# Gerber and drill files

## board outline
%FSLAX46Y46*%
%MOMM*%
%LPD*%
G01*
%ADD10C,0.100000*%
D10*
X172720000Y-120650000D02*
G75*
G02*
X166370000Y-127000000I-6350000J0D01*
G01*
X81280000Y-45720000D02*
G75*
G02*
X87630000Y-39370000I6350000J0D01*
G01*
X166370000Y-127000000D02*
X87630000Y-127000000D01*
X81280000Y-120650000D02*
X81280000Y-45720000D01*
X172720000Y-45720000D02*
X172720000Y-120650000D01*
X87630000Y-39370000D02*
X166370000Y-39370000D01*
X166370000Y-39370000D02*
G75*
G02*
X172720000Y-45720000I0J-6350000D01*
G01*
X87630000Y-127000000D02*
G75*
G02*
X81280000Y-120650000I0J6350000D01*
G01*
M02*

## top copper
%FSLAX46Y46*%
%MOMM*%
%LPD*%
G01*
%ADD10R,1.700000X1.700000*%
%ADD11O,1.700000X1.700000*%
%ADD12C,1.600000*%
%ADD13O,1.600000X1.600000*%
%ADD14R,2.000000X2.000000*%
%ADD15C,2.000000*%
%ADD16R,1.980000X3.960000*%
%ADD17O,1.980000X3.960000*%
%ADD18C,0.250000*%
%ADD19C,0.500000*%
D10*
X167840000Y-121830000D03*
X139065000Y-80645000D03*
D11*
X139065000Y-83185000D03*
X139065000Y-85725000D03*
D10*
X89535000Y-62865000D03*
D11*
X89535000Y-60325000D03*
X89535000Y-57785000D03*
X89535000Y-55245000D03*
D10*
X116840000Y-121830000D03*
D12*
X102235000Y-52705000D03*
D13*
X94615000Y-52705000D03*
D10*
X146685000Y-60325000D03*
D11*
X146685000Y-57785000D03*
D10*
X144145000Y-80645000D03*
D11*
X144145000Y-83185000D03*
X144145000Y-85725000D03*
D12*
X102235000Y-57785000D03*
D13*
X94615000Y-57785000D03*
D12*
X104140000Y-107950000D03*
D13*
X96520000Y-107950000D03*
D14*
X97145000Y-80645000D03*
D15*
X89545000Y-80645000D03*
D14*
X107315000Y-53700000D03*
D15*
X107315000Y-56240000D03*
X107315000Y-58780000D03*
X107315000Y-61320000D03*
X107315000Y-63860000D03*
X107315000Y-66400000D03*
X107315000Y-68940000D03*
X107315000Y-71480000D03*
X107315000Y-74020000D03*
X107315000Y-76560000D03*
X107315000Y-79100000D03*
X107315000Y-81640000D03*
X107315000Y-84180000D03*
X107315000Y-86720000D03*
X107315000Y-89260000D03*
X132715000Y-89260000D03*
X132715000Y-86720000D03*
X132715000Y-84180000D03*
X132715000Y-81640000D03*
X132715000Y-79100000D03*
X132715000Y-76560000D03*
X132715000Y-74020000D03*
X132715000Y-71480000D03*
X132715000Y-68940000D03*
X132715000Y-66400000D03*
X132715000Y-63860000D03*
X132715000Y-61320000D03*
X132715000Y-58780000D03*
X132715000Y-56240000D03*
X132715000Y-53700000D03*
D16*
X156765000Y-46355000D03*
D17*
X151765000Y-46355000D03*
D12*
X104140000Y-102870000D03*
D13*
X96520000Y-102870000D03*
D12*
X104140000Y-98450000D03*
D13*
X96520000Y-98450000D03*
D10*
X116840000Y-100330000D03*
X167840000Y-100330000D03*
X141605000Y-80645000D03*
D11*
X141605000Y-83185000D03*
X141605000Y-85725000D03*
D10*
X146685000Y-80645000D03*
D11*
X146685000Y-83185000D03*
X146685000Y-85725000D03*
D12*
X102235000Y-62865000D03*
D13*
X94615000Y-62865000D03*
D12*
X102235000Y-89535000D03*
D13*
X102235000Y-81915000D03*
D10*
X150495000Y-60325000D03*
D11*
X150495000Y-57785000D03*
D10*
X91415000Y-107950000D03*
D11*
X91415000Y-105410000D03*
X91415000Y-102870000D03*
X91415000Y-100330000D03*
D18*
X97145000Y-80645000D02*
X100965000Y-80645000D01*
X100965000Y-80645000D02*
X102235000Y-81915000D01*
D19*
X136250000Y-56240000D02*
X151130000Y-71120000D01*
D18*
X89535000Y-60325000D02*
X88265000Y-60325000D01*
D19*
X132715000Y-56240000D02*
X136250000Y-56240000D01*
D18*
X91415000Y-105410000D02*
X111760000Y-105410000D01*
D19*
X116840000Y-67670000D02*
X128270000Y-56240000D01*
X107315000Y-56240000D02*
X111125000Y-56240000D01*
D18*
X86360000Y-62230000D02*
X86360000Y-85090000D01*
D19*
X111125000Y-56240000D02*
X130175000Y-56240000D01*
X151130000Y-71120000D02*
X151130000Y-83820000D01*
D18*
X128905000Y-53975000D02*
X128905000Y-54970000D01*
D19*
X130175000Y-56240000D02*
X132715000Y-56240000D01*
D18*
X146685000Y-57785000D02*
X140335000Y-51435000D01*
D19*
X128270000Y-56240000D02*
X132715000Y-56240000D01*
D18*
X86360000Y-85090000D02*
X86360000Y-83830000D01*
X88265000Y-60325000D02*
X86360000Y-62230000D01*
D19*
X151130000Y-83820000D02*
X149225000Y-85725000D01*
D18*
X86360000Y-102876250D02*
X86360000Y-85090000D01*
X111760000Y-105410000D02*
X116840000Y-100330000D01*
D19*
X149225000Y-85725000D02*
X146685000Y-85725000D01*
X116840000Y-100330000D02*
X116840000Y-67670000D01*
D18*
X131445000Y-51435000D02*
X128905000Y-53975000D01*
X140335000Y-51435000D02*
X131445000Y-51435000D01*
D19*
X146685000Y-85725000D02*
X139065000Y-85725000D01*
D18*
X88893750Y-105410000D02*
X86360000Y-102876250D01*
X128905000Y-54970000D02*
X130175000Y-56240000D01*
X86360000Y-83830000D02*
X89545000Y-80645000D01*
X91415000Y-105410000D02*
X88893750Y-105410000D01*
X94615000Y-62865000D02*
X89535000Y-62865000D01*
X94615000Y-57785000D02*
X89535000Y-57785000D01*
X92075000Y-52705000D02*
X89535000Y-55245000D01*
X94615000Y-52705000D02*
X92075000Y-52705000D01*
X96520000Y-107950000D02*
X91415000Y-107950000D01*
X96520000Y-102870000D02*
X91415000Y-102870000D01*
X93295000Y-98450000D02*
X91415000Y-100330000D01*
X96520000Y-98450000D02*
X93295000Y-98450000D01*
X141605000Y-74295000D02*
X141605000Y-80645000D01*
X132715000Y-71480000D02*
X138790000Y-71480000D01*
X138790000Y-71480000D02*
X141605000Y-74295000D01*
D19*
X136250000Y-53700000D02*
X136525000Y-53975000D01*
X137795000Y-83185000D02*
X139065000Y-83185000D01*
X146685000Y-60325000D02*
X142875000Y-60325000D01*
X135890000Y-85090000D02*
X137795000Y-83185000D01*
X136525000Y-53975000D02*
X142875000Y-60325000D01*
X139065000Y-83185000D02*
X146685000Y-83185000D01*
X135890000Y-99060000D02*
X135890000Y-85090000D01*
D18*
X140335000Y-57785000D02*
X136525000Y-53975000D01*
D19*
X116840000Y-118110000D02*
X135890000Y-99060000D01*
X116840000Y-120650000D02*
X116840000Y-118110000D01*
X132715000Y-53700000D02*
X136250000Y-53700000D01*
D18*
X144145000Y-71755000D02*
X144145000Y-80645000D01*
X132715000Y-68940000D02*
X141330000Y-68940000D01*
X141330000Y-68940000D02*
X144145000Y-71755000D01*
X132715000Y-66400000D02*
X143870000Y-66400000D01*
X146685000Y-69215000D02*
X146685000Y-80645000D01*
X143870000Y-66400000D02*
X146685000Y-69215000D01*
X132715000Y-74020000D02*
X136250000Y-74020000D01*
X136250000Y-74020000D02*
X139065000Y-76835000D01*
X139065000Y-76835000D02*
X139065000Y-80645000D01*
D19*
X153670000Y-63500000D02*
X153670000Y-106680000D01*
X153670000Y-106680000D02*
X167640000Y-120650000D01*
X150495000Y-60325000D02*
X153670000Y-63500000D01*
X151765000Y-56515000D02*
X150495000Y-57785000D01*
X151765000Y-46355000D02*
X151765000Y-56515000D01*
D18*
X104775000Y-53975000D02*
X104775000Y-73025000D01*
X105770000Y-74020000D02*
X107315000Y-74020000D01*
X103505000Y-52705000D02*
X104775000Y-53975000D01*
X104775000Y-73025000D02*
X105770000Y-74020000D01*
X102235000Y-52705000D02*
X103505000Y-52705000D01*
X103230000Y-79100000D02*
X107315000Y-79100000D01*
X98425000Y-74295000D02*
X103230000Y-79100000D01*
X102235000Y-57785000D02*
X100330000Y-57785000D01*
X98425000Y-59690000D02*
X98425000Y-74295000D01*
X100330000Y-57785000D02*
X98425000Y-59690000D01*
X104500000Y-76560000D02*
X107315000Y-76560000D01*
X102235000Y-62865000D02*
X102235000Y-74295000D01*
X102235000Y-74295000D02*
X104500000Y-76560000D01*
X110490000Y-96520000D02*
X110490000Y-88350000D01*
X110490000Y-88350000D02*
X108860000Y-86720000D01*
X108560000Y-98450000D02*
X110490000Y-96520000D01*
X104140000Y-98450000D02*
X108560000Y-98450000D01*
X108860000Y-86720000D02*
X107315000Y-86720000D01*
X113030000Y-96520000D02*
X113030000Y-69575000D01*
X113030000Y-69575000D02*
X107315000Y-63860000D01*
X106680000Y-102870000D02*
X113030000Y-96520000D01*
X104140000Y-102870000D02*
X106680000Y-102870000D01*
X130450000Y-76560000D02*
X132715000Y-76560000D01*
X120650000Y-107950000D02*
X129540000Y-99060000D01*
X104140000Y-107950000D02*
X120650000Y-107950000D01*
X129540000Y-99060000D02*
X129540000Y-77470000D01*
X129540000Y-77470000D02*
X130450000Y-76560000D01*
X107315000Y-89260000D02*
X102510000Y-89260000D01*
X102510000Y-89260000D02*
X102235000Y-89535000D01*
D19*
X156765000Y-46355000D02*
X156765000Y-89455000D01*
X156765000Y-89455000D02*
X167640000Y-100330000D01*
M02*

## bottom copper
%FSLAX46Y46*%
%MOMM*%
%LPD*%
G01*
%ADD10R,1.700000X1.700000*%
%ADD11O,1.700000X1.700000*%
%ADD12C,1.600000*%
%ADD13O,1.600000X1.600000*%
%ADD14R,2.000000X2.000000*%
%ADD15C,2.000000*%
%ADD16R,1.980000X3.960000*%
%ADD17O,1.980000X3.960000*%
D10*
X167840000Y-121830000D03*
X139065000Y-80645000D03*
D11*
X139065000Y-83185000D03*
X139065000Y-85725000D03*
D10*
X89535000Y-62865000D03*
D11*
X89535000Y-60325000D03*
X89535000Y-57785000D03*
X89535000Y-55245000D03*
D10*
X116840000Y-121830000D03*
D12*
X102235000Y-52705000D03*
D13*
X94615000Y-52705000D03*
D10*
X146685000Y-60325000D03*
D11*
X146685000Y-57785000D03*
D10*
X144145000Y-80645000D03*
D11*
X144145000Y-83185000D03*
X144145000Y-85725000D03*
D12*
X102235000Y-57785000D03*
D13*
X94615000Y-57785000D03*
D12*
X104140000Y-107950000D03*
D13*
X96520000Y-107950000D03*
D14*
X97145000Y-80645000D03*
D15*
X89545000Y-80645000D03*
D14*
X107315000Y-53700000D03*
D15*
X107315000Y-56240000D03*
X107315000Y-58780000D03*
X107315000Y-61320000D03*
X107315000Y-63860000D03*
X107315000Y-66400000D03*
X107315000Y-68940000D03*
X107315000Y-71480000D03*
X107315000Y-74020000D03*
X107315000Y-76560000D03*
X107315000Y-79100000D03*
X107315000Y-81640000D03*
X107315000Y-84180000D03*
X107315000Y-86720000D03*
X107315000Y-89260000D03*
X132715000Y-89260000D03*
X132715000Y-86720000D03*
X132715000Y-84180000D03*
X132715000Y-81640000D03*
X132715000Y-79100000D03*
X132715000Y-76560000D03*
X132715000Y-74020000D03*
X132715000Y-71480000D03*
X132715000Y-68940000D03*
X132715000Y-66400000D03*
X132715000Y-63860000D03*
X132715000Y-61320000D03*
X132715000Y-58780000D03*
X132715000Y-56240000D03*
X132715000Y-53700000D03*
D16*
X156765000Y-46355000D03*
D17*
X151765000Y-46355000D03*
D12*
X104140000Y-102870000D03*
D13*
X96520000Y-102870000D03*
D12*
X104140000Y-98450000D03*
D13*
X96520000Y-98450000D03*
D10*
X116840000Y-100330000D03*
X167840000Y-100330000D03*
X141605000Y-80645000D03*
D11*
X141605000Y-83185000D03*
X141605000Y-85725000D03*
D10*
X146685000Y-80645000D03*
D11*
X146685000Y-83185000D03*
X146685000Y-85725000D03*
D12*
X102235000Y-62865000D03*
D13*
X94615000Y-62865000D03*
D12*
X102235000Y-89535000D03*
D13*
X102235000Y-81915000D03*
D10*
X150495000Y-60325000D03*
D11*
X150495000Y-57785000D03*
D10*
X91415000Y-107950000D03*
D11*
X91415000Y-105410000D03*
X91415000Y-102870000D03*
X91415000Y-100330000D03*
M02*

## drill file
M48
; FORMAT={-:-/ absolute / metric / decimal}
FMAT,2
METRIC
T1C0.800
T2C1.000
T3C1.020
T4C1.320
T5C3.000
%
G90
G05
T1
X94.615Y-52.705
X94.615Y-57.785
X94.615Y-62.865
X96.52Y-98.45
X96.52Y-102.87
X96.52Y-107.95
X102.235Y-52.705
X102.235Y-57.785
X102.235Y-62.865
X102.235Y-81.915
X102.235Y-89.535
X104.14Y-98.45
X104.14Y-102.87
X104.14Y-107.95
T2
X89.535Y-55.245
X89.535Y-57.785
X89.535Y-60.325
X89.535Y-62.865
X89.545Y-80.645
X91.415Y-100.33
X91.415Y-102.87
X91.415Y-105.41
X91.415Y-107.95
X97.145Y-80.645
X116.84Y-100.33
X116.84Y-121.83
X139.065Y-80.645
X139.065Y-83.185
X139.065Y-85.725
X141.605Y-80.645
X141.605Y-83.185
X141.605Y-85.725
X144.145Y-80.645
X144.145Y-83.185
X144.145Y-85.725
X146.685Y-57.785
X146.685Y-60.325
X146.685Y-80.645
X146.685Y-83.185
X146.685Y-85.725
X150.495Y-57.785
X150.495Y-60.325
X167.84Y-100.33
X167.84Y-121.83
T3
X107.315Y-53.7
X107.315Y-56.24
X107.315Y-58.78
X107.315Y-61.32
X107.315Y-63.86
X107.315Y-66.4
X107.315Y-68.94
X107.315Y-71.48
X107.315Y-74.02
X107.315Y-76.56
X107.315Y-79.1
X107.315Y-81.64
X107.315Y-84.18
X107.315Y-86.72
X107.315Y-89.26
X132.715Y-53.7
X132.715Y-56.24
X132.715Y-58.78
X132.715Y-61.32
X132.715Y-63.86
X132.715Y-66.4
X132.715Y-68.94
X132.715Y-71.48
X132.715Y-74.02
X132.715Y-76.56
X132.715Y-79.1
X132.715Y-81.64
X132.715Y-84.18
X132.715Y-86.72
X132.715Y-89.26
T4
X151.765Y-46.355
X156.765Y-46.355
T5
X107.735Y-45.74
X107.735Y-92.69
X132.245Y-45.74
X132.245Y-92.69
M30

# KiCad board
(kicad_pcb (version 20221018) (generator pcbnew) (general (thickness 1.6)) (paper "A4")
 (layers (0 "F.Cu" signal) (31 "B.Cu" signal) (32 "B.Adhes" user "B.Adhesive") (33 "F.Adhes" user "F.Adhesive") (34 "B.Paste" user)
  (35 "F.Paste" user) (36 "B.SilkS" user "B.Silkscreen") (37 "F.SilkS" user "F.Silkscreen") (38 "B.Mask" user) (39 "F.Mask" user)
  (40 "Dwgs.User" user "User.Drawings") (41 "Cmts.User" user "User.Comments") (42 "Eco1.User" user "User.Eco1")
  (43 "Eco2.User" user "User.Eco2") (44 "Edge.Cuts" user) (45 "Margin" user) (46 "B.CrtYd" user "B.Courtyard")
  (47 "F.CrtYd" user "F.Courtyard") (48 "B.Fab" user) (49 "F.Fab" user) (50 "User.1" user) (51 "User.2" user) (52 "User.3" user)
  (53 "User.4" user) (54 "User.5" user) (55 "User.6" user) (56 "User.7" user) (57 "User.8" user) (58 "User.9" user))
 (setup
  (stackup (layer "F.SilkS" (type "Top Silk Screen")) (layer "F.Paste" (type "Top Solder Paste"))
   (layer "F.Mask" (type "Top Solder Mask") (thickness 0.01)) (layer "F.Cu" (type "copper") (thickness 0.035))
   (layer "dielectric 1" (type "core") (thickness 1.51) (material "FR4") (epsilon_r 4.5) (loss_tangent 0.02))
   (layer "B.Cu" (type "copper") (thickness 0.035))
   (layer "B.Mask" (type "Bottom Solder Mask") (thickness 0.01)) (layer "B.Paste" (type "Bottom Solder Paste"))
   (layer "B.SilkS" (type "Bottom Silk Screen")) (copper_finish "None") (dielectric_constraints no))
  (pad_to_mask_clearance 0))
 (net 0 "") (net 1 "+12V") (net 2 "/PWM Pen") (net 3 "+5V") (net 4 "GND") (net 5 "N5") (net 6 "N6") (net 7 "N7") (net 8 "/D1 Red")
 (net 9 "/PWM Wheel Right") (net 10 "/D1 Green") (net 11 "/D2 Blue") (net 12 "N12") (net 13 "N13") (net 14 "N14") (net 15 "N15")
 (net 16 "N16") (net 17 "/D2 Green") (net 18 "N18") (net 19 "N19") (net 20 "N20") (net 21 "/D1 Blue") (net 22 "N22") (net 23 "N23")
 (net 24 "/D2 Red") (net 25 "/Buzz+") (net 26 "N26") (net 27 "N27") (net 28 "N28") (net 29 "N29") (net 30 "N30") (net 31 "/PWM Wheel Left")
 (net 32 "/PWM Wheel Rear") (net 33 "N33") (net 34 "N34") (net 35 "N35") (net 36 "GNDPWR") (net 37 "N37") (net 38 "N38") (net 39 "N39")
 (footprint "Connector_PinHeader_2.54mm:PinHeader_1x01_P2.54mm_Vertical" (layer "F.Cu") (at 167.84 121.83 180)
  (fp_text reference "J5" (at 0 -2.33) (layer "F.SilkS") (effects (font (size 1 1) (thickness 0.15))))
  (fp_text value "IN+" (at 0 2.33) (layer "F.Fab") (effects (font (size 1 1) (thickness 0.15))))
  (pad "1" thru_hole rect (at 0 0 180) (size 1.7 1.7) (drill 1) (layers "*.Cu" "*.Mask") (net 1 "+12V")))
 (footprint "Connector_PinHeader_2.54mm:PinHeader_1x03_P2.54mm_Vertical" (layer "F.Cu") (at 139.065 80.645)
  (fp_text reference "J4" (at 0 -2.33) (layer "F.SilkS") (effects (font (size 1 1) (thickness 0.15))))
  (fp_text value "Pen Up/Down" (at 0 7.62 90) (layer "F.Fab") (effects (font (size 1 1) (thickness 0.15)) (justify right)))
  (pad "1" thru_hole rect (at 0 0) (size 1.7 1.7) (drill 1) (layers "*.Cu" "*.Mask") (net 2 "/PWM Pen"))
  (pad "2" thru_hole oval (at 0 2.54) (size 1.7 1.7) (drill 1) (layers "*.Cu" "*.Mask") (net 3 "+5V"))
  (pad "3" thru_hole oval (at 0 5.08) (size 1.7 1.7) (drill 1) (layers "*.Cu" "*.Mask") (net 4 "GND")))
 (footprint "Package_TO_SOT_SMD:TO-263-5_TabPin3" (layer "F.Cu") (at 143.395 110.255)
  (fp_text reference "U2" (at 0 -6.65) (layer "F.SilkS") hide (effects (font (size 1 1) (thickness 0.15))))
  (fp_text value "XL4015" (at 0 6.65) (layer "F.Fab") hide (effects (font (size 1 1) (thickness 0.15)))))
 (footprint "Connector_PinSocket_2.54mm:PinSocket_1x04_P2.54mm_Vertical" (layer "F.Cu") (at 89.535 62.865 180)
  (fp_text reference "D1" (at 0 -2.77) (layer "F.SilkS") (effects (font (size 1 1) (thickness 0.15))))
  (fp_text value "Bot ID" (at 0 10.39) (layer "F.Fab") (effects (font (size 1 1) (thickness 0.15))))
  (pad "1" thru_hole rect (at 0 0 180) (size 1.7 1.7) (drill 1) (layers "*.Cu" "*.Mask") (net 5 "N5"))
  (pad "2" thru_hole oval (at 0 2.54 180) (size 1.7 1.7) (drill 1) (layers "*.Cu" "*.Mask") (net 4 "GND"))
  (pad "3" thru_hole oval (at 0 5.08 180) (size 1.7 1.7) (drill 1) (layers "*.Cu" "*.Mask") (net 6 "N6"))
  (pad "4" thru_hole oval (at 0 7.62 180) (size 1.7 1.7) (drill 1) (layers "*.Cu" "*.Mask") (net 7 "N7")))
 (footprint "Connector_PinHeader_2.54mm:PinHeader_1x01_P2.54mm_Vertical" (layer "F.Cu") (at 116.84 121.83 180)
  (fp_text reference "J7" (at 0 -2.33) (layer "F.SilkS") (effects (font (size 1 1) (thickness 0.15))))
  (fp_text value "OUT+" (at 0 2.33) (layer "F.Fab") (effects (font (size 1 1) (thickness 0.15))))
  (pad "1" thru_hole rect (at 0 0 180) (size 1.7 1.7) (drill 1) (layers "*.Cu" "*.Mask") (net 3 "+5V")))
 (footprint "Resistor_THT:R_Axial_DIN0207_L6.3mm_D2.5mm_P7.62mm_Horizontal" (layer "F.Cu") (at 102.235 52.705 180)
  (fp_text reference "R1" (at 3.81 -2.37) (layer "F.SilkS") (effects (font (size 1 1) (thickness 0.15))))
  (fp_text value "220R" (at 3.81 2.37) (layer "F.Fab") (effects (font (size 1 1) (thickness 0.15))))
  (pad "1" thru_hole circle (at 0 0 180) (size 1.6 1.6) (drill 0.8) (layers "*.Cu" "*.Mask") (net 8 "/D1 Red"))
  (pad "2" thru_hole oval (at 7.62 0 180) (size 1.6 1.6) (drill 0.8) (layers "*.Cu" "*.Mask") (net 7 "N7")))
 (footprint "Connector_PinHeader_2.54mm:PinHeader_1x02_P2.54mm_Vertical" (layer "F.Cu") (at 146.685 60.325 180)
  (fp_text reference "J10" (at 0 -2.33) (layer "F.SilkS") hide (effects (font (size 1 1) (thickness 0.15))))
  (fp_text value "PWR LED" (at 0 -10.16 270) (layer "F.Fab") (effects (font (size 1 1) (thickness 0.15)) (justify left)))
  (pad "1" thru_hole rect (at 0 0 180) (size 1.7 1.7) (drill 1) (layers "*.Cu" "*.Mask") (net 3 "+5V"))
  (pad "2" thru_hole oval (at 0 2.54 180) (size 1.7 1.7) (drill 1) (layers "*.Cu" "*.Mask") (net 4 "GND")))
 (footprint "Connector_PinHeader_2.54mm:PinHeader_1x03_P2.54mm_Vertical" (layer "F.Cu") (at 144.145 80.645)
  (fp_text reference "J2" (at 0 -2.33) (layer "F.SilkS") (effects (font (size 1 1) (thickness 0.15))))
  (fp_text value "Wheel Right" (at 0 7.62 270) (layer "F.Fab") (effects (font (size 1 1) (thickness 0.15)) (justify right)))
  (pad "1" thru_hole rect (at 0 0) (size 1.7 1.7) (drill 1) (layers "*.Cu" "*.Mask") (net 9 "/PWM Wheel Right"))
  (pad "2" thru_hole oval (at 0 2.54) (size 1.7 1.7) (drill 1) (layers "*.Cu" "*.Mask") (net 3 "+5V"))
  (pad "3" thru_hole oval (at 0 5.08) (size 1.7 1.7) (drill 1) (layers "*.Cu" "*.Mask") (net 4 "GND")))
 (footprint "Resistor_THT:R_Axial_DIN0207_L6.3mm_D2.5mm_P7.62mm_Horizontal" (layer "F.Cu") (at 102.235 57.785 180)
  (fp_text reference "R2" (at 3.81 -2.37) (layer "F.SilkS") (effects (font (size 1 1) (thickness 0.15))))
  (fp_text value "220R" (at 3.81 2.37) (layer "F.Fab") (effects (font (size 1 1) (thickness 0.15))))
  (pad "1" thru_hole circle (at 0 0 180) (size 1.6 1.6) (drill 0.8) (layers "*.Cu" "*.Mask") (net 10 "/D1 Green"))
  (pad "2" thru_hole oval (at 7.62 0 180) (size 1.6 1.6) (drill 0.8) (layers "*.Cu" "*.Mask") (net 6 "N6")))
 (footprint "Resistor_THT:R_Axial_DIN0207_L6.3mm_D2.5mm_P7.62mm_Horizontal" (layer "F.Cu") (at 104.14 107.95 180)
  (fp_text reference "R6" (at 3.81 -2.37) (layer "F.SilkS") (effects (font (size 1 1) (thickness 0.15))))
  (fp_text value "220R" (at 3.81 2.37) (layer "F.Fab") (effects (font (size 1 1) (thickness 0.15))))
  (pad "1" thru_hole circle (at 0 0 180) (size 1.6 1.6) (drill 0.8) (layers "*.Cu" "*.Mask") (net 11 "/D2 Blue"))
  (pad "2" thru_hole oval (at 7.62 0 180) (size 1.6 1.6) (drill 0.8) (layers "*.Cu" "*.Mask") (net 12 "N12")))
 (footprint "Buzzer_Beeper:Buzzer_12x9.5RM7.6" (layer "F.Cu") (at 97.145 80.645 180)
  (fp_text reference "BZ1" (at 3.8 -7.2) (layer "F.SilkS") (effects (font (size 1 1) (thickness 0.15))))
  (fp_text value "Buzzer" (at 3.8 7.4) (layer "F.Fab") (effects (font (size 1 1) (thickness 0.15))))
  (pad "1" thru_hole rect (at 0 0 180) (size 2 2) (drill 1) (layers "*.Cu" "*.Mask") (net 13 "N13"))
  (pad "2" thru_hole circle (at 7.6 0 180) (size 2 2) (drill 1) (layers "*.Cu" "*.Mask") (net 4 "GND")))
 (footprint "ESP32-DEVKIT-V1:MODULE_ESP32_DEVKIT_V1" (layer "F.Cu") (at 120.015 69.215)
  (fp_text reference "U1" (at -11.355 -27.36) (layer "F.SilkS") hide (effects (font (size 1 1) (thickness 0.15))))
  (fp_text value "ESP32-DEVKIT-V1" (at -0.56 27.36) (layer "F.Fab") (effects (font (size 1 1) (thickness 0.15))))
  (pad "" np_thru_hole circle (at -12.28 -23.475) (size 3 3) (drill 3) (layers "*.Cu" "*.Mask"))
  (pad "" np_thru_hole circle (at -12.28 23.475) (size 3 3) (drill 3) (layers "*.Cu" "*.Mask"))
  (pad "" np_thru_hole circle (at 12.23 -23.475) (size 3 3) (drill 3) (layers "*.Cu" "*.Mask"))
  (pad "" np_thru_hole circle (at 12.23 23.475) (size 3 3) (drill 3) (layers "*.Cu" "*.Mask"))
  (pad "1" thru_hole rect (at -12.7 -15.515) (size 2 2) (drill 1.02) (layers "*.Cu" "*.Mask") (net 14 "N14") (solder_mask_margin 0.102))
  (pad "2" thru_hole circle (at -12.7 -12.975) (size 2 2) (drill 1.02) (layers "*.Cu" "*.Mask") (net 4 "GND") (solder_mask_margin 0.102))
  (pad "3" thru_hole circle (at -12.7 -10.435) (size 2 2) (drill 1.02) (layers "*.Cu" "*.Mask") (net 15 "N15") (solder_mask_margin 0.102))
  (pad "4" thru_hole circle (at -12.7 -7.895) (size 2 2) (drill 1.02) (layers "*.Cu" "*.Mask") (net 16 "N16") (solder_mask_margin 0.102))
  (pad "5" thru_hole circle (at -12.7 -5.355) (size 2 2) (drill 1.02) (layers "*.Cu" "*.Mask") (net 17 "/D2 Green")
   (solder_mask_margin 0.102))
  (pad "6" thru_hole circle (at -12.7 -2.815) (size 2 2) (drill 1.02) (layers "*.Cu" "*.Mask") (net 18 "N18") (solder_mask_margin 0.102))
  (pad "7" thru_hole circle (at -12.7 -0.275) (size 2 2) (drill 1.02) (layers "*.Cu" "*.Mask") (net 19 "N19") (solder_mask_margin 0.102))
  (pad "8" thru_hole circle (at -12.7 2.265) (size 2 2) (drill 1.02) (layers "*.Cu" "*.Mask") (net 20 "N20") (solder_mask_margin 0.102))
  (pad "9" thru_hole circle (at -12.7 4.805) (size 2 2) (drill 1.02) (layers "*.Cu" "*.Mask") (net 8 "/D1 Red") (solder_mask_margin 0.102))
  (pad "10" thru_hole circle (at -12.7 7.345) (size 2 2) (drill 1.02) (layers "*.Cu" "*.Mask") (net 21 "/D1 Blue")
   (solder_mask_margin 0.102))
  (pad "11" thru_hole circle (at -12.7 9.885) (size 2 2) (drill 1.02) (layers "*.Cu" "*.Mask") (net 10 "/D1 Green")
   (solder_mask_margin 0.102))
  (pad "12" thru_hole circle (at -12.7 12.425) (size 2 2) (drill 1.02) (layers "*.Cu" "*.Mask") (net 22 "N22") (solder_mask_margin 0.102))
  (pad "13" thru_hole circle (at -12.7 14.965) (size 2 2) (drill 1.02) (layers "*.Cu" "*.Mask") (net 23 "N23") (solder_mask_margin 0.102))
  (pad "14" thru_hole circle (at -12.7 17.505) (size 2 2) (drill 1.02) (layers "*.Cu" "*.Mask") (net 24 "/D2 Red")
   (solder_mask_margin 0.102))
  (pad "15" thru_hole circle (at -12.7 20.045) (size 2 2) (drill 1.02) (layers "*.Cu" "*.Mask") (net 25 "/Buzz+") (solder_mask_margin 0.102))
  (pad "16" thru_hole circle (at 12.7 20.045) (size 2 2) (drill 1.02) (layers "*.Cu" "*.Mask") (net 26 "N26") (solder_mask_margin 0.102))
  (pad "17" thru_hole circle (at 12.7 17.505) (size 2 2) (drill 1.02) (layers "*.Cu" "*.Mask") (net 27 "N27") (solder_mask_margin 0.102))
  (pad "18" thru_hole circle (at 12.7 14.965) (size 2 2) (drill 1.02) (layers "*.Cu" "*.Mask") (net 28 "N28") (solder_mask_margin 0.102))
  (pad "19" thru_hole circle (at 12.7 12.425) (size 2 2) (drill 1.02) (layers "*.Cu" "*.Mask") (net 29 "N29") (solder_mask_margin 0.102))
  (pad "20" thru_hole circle (at 12.7 9.885) (size 2 2) (drill 1.02) (layers "*.Cu" "*.Mask") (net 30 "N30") (solder_mask_margin 0.102))
  (pad "21" thru_hole circle (at 12.7 7.345) (size 2 2) (drill 1.02) (layers "*.Cu" "*.Mask") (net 11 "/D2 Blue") (solder_mask_margin 0.102))
  (pad "22" thru_hole circle (at 12.7 4.805) (size 2 2) (drill 1.02) (layers "*.Cu" "*.Mask") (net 2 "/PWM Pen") (solder_mask_margin 0.102))
  (pad "23" thru_hole circle (at 12.7 2.265) (size 2 2) (drill 1.02) (layers "*.Cu" "*.Mask") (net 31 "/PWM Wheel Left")
   (solder_mask_margin 0.102))
  (pad "24" thru_hole circle (at 12.7 -0.275) (size 2 2) (drill 1.02) (layers "*.Cu" "*.Mask") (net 9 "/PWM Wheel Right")
   (solder_mask_margin 0.102))
  (pad "25" thru_hole circle (at 12.7 -2.815) (size 2 2) (drill 1.02) (layers "*.Cu" "*.Mask") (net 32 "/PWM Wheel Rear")
   (solder_mask_margin 0.102))
  (pad "26" thru_hole circle (at 12.7 -5.355) (size 2 2) (drill 1.02) (layers "*.Cu" "*.Mask") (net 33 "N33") (solder_mask_margin 0.102))
  (pad "27" thru_hole circle (at 12.7 -7.895) (size 2 2) (drill 1.02) (layers "*.Cu" "*.Mask") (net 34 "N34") (solder_mask_margin 0.102))
  (pad "28" thru_hole circle (at 12.7 -10.435) (size 2 2) (drill 1.02) (layers "*.Cu" "*.Mask") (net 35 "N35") (solder_mask_margin 0.102))
  (pad "29" thru_hole circle (at 12.7 -12.975) (size 2 2) (drill 1.02) (layers "*.Cu" "*.Mask") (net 4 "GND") (solder_mask_margin 0.102))
  (pad "30" thru_hole circle (at 12.7 -15.515) (size 2 2) (drill 1.02) (layers "*.Cu" "*.Mask") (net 3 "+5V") (solder_mask_margin 0.102)))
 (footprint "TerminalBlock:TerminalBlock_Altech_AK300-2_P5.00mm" (layer "F.Cu") (at 156.765 46.355 180)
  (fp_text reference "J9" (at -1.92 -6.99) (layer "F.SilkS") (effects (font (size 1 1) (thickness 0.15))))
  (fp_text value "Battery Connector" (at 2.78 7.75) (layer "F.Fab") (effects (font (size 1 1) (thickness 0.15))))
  (pad "1" thru_hole rect (at 0 0 180) (size 1.98 3.96) (drill 1.32) (layers "*.Cu" "*.Mask") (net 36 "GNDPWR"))
  (pad "2" thru_hole oval (at 5 0 180) (size 1.98 3.96) (drill 1.32) (layers "*.Cu" "*.Mask") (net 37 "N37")))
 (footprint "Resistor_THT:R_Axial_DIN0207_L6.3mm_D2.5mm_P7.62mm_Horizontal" (layer "F.Cu") (at 104.14 102.87 180)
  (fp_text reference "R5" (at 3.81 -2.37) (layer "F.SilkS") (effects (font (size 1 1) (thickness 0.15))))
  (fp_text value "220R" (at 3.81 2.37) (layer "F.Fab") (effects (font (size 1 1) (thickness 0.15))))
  (pad "1" thru_hole circle (at 0 0 180) (size 1.6 1.6) (drill 0.8) (layers "*.Cu" "*.Mask") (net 17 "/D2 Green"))
  (pad "2" thru_hole oval (at 7.62 0 180) (size 1.6 1.6) (drill 0.8) (layers "*.Cu" "*.Mask") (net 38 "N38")))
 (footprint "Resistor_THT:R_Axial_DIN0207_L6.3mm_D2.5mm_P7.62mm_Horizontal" (layer "F.Cu") (at 104.14 98.45 180)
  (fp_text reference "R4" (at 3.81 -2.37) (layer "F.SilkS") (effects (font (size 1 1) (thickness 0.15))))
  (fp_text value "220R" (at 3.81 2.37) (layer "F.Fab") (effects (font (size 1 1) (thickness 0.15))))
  (pad "1" thru_hole circle (at 0 0 180) (size 1.6 1.6) (drill 0.8) (layers "*.Cu" "*.Mask") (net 24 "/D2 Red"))
  (pad "2" thru_hole oval (at 7.62 0 180) (size 1.6 1.6) (drill 0.8) (layers "*.Cu" "*.Mask") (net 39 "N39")))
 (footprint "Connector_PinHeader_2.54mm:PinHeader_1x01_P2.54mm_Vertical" (layer "F.Cu") (at 116.84 100.33 180)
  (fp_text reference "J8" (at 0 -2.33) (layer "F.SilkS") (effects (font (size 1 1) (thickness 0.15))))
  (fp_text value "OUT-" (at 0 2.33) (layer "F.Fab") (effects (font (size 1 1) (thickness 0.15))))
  (pad "1" thru_hole rect (at 0 0 180) (size 1.7 1.7) (drill 1) (layers "*.Cu" "*.Mask") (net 4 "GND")))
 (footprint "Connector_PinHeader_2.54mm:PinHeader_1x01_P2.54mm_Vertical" (layer "F.Cu") (at 167.84 100.33 180)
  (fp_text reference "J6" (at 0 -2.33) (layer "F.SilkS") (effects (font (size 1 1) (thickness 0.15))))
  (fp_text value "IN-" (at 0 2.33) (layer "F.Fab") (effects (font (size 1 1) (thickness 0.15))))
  (pad "1" thru_hole rect (at 0 0 180) (size 1.7 1.7) (drill 1) (layers "*.Cu" "*.Mask") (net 36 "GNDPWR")))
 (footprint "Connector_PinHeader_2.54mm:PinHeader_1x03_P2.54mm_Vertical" (layer "F.Cu") (at 141.605 80.645)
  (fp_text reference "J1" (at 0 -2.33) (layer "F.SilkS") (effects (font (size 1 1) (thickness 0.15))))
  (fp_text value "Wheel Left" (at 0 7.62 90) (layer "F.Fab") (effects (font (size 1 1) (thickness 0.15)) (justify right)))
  (pad "1" thru_hole rect (at 0 0) (size 1.7 1.7) (drill 1) (layers "*.Cu" "*.Mask") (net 31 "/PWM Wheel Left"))
  (pad "2" thru_hole oval (at 0 2.54) (size 1.7 1.7) (drill 1) (layers "*.Cu" "*.Mask") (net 3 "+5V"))
  (pad "3" thru_hole oval (at 0 5.08) (size 1.7 1.7) (drill 1) (layers "*.Cu" "*.Mask") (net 4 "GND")))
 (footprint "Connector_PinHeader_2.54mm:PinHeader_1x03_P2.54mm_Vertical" (layer "F.Cu") (at 146.685 80.645)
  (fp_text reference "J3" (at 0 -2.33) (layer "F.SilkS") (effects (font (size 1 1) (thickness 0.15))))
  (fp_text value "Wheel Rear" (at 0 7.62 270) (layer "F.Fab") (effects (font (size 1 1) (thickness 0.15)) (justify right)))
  (pad "1" thru_hole rect (at 0 0) (size 1.7 1.7) (drill 1) (layers "*.Cu" "*.Mask") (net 32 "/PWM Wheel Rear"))
  (pad "2" thru_hole oval (at 0 2.54) (size 1.7 1.7) (drill 1) (layers "*.Cu" "*.Mask") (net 3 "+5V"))
  (pad "3" thru_hole oval (at 0 5.08) (size 1.7 1.7) (drill 1) (layers "*.Cu" "*.Mask") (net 4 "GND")))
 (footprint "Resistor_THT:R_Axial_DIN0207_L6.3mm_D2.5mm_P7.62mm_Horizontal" (layer "F.Cu") (at 102.235 62.865 180)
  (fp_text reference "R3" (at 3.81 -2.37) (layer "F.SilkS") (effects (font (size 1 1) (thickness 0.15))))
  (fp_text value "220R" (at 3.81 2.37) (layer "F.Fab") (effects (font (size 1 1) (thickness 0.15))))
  (pad "1" thru_hole circle (at 0 0 180) (size 1.6 1.6) (drill 0.8) (layers "*.Cu" "*.Mask") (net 21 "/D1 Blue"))
  (pad "2" thru_hole oval (at 7.62 0 180) (size 1.6 1.6) (drill 0.8) (layers "*.Cu" "*.Mask") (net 5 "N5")))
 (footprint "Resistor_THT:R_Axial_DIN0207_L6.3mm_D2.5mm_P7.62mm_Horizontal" (layer "F.Cu") (at 102.235 89.535 90)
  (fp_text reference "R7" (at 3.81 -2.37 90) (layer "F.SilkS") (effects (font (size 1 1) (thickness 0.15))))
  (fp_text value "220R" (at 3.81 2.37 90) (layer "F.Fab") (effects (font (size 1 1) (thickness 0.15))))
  (pad "1" thru_hole circle (at 0 0 90) (size 1.6 1.6) (drill 0.8) (layers "*.Cu" "*.Mask") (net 25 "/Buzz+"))
  (pad "2" thru_hole oval (at 7.62 0 90) (size 1.6 1.6) (drill 0.8) (layers "*.Cu" "*.Mask") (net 13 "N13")))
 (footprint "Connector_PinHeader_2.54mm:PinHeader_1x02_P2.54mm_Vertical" (layer "F.Cu") (at 150.495 60.325 180)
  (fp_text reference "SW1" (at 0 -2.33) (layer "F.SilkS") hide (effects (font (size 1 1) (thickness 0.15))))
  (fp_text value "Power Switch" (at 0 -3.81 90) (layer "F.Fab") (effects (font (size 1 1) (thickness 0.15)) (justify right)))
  (pad "1" thru_hole rect (at 0 0 180) (size 1.7 1.7) (drill 1) (layers "*.Cu" "*.Mask") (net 1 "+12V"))
  (pad "2" thru_hole oval (at 0 2.54 180) (size 1.7 1.7) (drill 1) (layers "*.Cu" "*.Mask") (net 37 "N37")))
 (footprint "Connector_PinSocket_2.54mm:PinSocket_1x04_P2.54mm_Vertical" (layer "F.Cu") (at 91.415 107.95 180)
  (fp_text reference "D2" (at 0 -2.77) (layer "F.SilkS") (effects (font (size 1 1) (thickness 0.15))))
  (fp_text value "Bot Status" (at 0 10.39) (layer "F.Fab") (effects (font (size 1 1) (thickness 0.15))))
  (pad "1" thru_hole rect (at 0 0 180) (size 1.7 1.7) (drill 1) (layers "*.Cu" "*.Mask") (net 12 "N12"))
  (pad "2" thru_hole oval (at 0 2.54 180) (size 1.7 1.7) (drill 1) (layers "*.Cu" "*.Mask") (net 4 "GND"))
  (pad "3" thru_hole oval (at 0 5.08 180) (size 1.7 1.7) (drill 1) (layers "*.Cu" "*.Mask") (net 38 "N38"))
  (pad "4" thru_hole oval (at 0 7.62 180) (size 1.7 1.7) (drill 1) (layers "*.Cu" "*.Mask") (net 39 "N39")))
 (gr_arc (start 172.72 120.65) (mid 170.860128 125.140128) (end 166.37 127) (stroke (width 0.1) (type default)) (layer "Edge.Cuts"))
 (gr_arc (start 81.28 45.72) (mid 83.139872 41.229872) (end 87.63 39.37) (stroke (width 0.1) (type default)) (layer "Edge.Cuts"))
 (gr_line (start 166.37 127) (end 87.63 127) (stroke (width 0.1) (type default)) (layer "Edge.Cuts"))
 (gr_line (start 81.28 120.65) (end 81.28 45.72) (stroke (width 0.1) (type default)) (layer "Edge.Cuts"))
 (gr_line (start 172.72 45.72) (end 172.72 120.65) (stroke (width 0.1) (type default)) (layer "Edge.Cuts"))
 (gr_line (start 87.63 39.37) (end 166.37 39.37) (stroke (width 0.1) (type default)) (layer "Edge.Cuts"))
 (gr_arc (start 166.37 39.37) (mid 170.860128 41.229872) (end 172.72 45.72) (stroke (width 0.1) (type default)) (layer "Edge.Cuts"))
 (gr_arc (start 87.63 127) (mid 83.139872 125.140128) (end 81.28 120.65) (stroke (width 0.1) (type default)) (layer "Edge.Cuts"))
 (segment (start 97.145 80.645) (end 100.965 80.645) (width 0.25) (layer "F.Cu") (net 13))
 (segment (start 100.965 80.645) (end 102.235 81.915) (width 0.25) (layer "F.Cu") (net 13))
 (segment (start 136.25 56.24) (end 151.13 71.12) (width 0.5) (layer "F.Cu") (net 4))
 (segment (start 89.535 60.325) (end 88.265 60.325) (width 0.25) (layer "F.Cu") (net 4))
 (segment (start 132.715 56.24) (end 136.25 56.24) (width 0.5) (layer "F.Cu") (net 4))
 (segment (start 91.415 105.41) (end 111.76 105.41) (width 0.25) (layer "F.Cu") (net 4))
 (segment (start 116.84 67.67) (end 128.27 56.24) (width 0.5) (layer "F.Cu") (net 4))
 (segment (start 107.315 56.24) (end 111.125 56.24) (width 0.5) (layer "F.Cu") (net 4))
 (segment (start 86.36 62.23) (end 86.36 85.09) (width 0.25) (layer "F.Cu") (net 4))
 (segment (start 111.125 56.24) (end 130.175 56.24) (width 0.5) (layer "F.Cu") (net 4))
 (segment (start 151.13 71.12) (end 151.13 83.82) (width 0.5) (layer "F.Cu") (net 4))
 (segment (start 128.905 53.975) (end 128.905 54.97) (width 0.25) (layer "F.Cu") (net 4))
 (segment (start 130.175 56.24) (end 132.715 56.24) (width 0.5) (layer "F.Cu") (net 4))
 (segment (start 146.685 57.785) (end 140.335 51.435) (width 0.25) (layer "F.Cu") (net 4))
 (segment (start 128.27 56.24) (end 132.715 56.24) (width 0.5) (layer "F.Cu") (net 4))
 (segment (start 86.36 85.09) (end 86.36 83.83) (width 0.25) (layer "F.Cu") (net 4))
 (segment (start 88.265 60.325) (end 86.36 62.23) (width 0.25) (layer "F.Cu") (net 4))
 (segment (start 151.13 83.82) (end 149.225 85.725) (width 0.5) (layer "F.Cu") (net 4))
 (segment (start 86.36 102.87625) (end 86.36 85.09) (width 0.25) (layer "F.Cu") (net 4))
 (segment (start 111.76 105.41) (end 116.84 100.33) (width 0.25) (layer "F.Cu") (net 4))
 (segment (start 149.225 85.725) (end 146.685 85.725) (width 0.5) (layer "F.Cu") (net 4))
 (segment (start 116.84 100.33) (end 116.84 67.67) (width 0.5) (layer "F.Cu") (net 4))
 (segment (start 131.445 51.435) (end 128.905 53.975) (width 0.25) (layer "F.Cu") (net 4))
 (segment (start 140.335 51.435) (end 131.445 51.435) (width 0.25) (layer "F.Cu") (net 4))
 (segment (start 146.685 85.725) (end 139.065 85.725) (width 0.5) (layer "F.Cu") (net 4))
 (segment (start 88.89375 105.41) (end 86.36 102.87625) (width 0.25) (layer "F.Cu") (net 4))
 (segment (start 128.905 54.97) (end 130.175 56.24) (width 0.25) (layer "F.Cu") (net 4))
 (segment (start 86.36 83.83) (end 89.545 80.645) (width 0.25) (layer "F.Cu") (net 4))
 (segment (start 91.415 105.41) (end 88.89375 105.41) (width 0.25) (layer "F.Cu") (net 4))
 (segment (start 94.615 62.865) (end 89.535 62.865) (width 0.25) (layer "F.Cu") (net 5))
 (segment (start 94.615 57.785) (end 89.535 57.785) (width 0.25) (layer "F.Cu") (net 6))
 (segment (start 92.075 52.705) (end 89.535 55.245) (width 0.25) (layer "F.Cu") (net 7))
 (segment (start 94.615 52.705) (end 92.075 52.705) (width 0.25) (layer "F.Cu") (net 7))
 (segment (start 96.52 107.95) (end 91.415 107.95) (width 0.25) (layer "F.Cu") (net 12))
 (segment (start 96.52 102.87) (end 91.415 102.87) (width 0.25) (layer "F.Cu") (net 38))
 (segment (start 93.295 98.45) (end 91.415 100.33) (width 0.25) (layer "F.Cu") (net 39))
 (segment (start 96.52 98.45) (end 93.295 98.45) (width 0.25) (layer "F.Cu") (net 39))
 (segment (start 141.605 74.295) (end 141.605 80.645) (width 0.25) (layer "F.Cu") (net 31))
 (segment (start 132.715 71.48) (end 138.79 71.48) (width 0.25) (layer "F.Cu") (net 31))
 (segment (start 138.79 71.48) (end 141.605 74.295) (width 0.25) (layer "F.Cu") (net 31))
 (segment (start 136.25 53.7) (end 136.525 53.975) (width 0.5) (layer "F.Cu") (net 3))
 (segment (start 137.795 83.185) (end 139.065 83.185) (width 0.5) (layer "F.Cu") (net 3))
 (segment (start 146.685 60.325) (end 142.875 60.325) (width 0.5) (layer "F.Cu") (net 3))
 (segment (start 135.89 85.09) (end 137.795 83.185) (width 0.5) (layer "F.Cu") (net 3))
 (segment (start 136.525 53.975) (end 142.875 60.325) (width 0.5) (layer "F.Cu") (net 3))
 (segment (start 139.065 83.185) (end 146.685 83.185) (width 0.5) (layer "F.Cu") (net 3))
 (segment (start 135.89 99.06) (end 135.89 85.09) (width 0.5) (layer "F.Cu") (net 3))
 (segment (start 140.335 57.785) (end 136.525 53.975) (width 0.25) (layer "F.Cu") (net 3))
 (segment (start 116.84 118.11) (end 135.89 99.06) (width 0.5) (layer "F.Cu") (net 3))
 (segment (start 116.84 120.65) (end 116.84 118.11) (width 0.5) (layer "F.Cu") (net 3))
 (segment (start 132.715 53.7) (end 136.25 53.7) (width 0.5) (layer "F.Cu") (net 3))
 (segment (start 144.145 71.755) (end 144.145 80.645) (width 0.25) (layer "F.Cu") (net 9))
 (segment (start 132.715 68.94) (end 141.33 68.94) (width 0.25) (layer "F.Cu") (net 9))
 (segment (start 141.33 68.94) (end 144.145 71.755) (width 0.25) (layer "F.Cu") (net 9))
 (segment (start 132.715 66.4) (end 143.87 66.4) (width 0.25) (layer "F.Cu") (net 32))
 (segment (start 146.685 69.215) (end 146.685 80.645) (width 0.25) (layer "F.Cu") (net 32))
 (segment (start 143.87 66.4) (end 146.685 69.215) (width 0.25) (layer "F.Cu") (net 32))
 (segment (start 132.715 74.02) (end 136.25 74.02) (width 0.25) (layer "F.Cu") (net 2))
 (segment (start 136.25 74.02) (end 139.065 76.835) (width 0.25) (layer "F.Cu") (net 2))
 (segment (start 139.065 76.835) (end 139.065 80.645) (width 0.25) (layer "F.Cu") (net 2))
 (segment (start 153.67 63.5) (end 153.67 106.68) (width 0.5) (layer "F.Cu") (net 1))
 (segment (start 153.67 106.68) (end 167.64 120.65) (width 0.5) (layer "F.Cu") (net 1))
 (segment (start 150.495 60.325) (end 153.67 63.5) (width 0.5) (layer "F.Cu") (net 1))
 (segment (start 151.765 56.515) (end 150.495 57.785) (width 0.5) (layer "F.Cu") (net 37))
 (segment (start 151.765 46.355) (end 151.765 56.515) (width 0.5) (layer "F.Cu") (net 37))
 (segment (start 104.775 53.975) (end 104.775 73.025) (width 0.25) (layer "F.Cu") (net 8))
 (segment (start 105.77 74.02) (end 107.315 74.02) (width 0.25) (layer "F.Cu") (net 8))
 (segment (start 103.505 52.705) (end 104.775 53.975) (width 0.25) (layer "F.Cu") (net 8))
 (segment (start 104.775 73.025) (end 105.77 74.02) (width 0.25) (layer "F.Cu") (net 8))
 (segment (start 102.235 52.705) (end 103.505 52.705) (width 0.25) (layer "F.Cu") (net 8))
 (segment (start 103.23 79.1) (end 107.315 79.1) (width 0.25) (layer "F.Cu") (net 10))
 (segment (start 98.425 74.295) (end 103.23 79.1) (width 0.25) (layer "F.Cu") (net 10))
 (segment (start 102.235 57.785) (end 100.33 57.785) (width 0.25) (layer "F.Cu") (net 10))
 (segment (start 98.425 59.69) (end 98.425 74.295) (width 0.25) (layer "F.Cu") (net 10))
 (segment (start 100.33 57.785) (end 98.425 59.69) (width 0.25) (layer "F.Cu") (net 10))
 (segment (start 104.5 76.56) (end 107.315 76.56) (width 0.25) (layer "F.Cu") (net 21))
 (segment (start 102.235 62.865) (end 102.235 74.295) (width 0.25) (layer "F.Cu") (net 21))
 (segment (start 102.235 74.295) (end 104.5 76.56) (width 0.25) (layer "F.Cu") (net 21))
 (segment (start 110.49 96.52) (end 110.49 88.35) (width 0.25) (layer "F.Cu") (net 24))
 (segment (start 110.49 88.35) (end 108.86 86.72) (width 0.25) (layer "F.Cu") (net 24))
 (segment (start 108.56 98.45) (end 110.49 96.52) (width 0.25) (layer "F.Cu") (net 24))
 (segment (start 104.14 98.45) (end 108.56 98.45) (width 0.25) (layer "F.Cu") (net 24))
 (segment (start 108.86 86.72) (end 107.315 86.72) (width 0.25) (layer "F.Cu") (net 24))
 (segment (start 113.03 96.52) (end 113.03 69.575) (width 0.25) (layer "F.Cu") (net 17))
 (segment (start 113.03 69.575) (end 107.315 63.86) (width 0.25) (layer "F.Cu") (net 17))
 (segment (start 106.68 102.87) (end 113.03 96.52) (width 0.25) (layer "F.Cu") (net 17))
 (segment (start 104.14 102.87) (end 106.68 102.87) (width 0.25) (layer "F.Cu") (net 17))
 (segment (start 130.45 76.56) (end 132.715 76.56) (width 0.25) (layer "F.Cu") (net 11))
 (segment (start 120.65 107.95) (end 129.54 99.06) (width 0.25) (layer "F.Cu") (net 11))
 (segment (start 104.14 107.95) (end 120.65 107.95) (width 0.25) (layer "F.Cu") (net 11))
 (segment (start 129.54 99.06) (end 129.54 77.47) (width 0.25) (layer "F.Cu") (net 11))
 (segment (start 129.54 77.47) (end 130.45 76.56) (width 0.25) (layer "F.Cu") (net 11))
 (segment (start 107.315 89.26) (end 102.51 89.26) (width 0.25) (layer "F.Cu") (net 25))
 (segment (start 102.51 89.26) (end 102.235 89.535) (width 0.25) (layer "F.Cu") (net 25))
 (segment (start 156.765 46.355) (end 156.765 89.455) (width 0.5) (layer "F.Cu") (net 36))
 (segment (start 156.765 89.455) (end 167.64 100.33) (width 0.5) (layer "F.Cu") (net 36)))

